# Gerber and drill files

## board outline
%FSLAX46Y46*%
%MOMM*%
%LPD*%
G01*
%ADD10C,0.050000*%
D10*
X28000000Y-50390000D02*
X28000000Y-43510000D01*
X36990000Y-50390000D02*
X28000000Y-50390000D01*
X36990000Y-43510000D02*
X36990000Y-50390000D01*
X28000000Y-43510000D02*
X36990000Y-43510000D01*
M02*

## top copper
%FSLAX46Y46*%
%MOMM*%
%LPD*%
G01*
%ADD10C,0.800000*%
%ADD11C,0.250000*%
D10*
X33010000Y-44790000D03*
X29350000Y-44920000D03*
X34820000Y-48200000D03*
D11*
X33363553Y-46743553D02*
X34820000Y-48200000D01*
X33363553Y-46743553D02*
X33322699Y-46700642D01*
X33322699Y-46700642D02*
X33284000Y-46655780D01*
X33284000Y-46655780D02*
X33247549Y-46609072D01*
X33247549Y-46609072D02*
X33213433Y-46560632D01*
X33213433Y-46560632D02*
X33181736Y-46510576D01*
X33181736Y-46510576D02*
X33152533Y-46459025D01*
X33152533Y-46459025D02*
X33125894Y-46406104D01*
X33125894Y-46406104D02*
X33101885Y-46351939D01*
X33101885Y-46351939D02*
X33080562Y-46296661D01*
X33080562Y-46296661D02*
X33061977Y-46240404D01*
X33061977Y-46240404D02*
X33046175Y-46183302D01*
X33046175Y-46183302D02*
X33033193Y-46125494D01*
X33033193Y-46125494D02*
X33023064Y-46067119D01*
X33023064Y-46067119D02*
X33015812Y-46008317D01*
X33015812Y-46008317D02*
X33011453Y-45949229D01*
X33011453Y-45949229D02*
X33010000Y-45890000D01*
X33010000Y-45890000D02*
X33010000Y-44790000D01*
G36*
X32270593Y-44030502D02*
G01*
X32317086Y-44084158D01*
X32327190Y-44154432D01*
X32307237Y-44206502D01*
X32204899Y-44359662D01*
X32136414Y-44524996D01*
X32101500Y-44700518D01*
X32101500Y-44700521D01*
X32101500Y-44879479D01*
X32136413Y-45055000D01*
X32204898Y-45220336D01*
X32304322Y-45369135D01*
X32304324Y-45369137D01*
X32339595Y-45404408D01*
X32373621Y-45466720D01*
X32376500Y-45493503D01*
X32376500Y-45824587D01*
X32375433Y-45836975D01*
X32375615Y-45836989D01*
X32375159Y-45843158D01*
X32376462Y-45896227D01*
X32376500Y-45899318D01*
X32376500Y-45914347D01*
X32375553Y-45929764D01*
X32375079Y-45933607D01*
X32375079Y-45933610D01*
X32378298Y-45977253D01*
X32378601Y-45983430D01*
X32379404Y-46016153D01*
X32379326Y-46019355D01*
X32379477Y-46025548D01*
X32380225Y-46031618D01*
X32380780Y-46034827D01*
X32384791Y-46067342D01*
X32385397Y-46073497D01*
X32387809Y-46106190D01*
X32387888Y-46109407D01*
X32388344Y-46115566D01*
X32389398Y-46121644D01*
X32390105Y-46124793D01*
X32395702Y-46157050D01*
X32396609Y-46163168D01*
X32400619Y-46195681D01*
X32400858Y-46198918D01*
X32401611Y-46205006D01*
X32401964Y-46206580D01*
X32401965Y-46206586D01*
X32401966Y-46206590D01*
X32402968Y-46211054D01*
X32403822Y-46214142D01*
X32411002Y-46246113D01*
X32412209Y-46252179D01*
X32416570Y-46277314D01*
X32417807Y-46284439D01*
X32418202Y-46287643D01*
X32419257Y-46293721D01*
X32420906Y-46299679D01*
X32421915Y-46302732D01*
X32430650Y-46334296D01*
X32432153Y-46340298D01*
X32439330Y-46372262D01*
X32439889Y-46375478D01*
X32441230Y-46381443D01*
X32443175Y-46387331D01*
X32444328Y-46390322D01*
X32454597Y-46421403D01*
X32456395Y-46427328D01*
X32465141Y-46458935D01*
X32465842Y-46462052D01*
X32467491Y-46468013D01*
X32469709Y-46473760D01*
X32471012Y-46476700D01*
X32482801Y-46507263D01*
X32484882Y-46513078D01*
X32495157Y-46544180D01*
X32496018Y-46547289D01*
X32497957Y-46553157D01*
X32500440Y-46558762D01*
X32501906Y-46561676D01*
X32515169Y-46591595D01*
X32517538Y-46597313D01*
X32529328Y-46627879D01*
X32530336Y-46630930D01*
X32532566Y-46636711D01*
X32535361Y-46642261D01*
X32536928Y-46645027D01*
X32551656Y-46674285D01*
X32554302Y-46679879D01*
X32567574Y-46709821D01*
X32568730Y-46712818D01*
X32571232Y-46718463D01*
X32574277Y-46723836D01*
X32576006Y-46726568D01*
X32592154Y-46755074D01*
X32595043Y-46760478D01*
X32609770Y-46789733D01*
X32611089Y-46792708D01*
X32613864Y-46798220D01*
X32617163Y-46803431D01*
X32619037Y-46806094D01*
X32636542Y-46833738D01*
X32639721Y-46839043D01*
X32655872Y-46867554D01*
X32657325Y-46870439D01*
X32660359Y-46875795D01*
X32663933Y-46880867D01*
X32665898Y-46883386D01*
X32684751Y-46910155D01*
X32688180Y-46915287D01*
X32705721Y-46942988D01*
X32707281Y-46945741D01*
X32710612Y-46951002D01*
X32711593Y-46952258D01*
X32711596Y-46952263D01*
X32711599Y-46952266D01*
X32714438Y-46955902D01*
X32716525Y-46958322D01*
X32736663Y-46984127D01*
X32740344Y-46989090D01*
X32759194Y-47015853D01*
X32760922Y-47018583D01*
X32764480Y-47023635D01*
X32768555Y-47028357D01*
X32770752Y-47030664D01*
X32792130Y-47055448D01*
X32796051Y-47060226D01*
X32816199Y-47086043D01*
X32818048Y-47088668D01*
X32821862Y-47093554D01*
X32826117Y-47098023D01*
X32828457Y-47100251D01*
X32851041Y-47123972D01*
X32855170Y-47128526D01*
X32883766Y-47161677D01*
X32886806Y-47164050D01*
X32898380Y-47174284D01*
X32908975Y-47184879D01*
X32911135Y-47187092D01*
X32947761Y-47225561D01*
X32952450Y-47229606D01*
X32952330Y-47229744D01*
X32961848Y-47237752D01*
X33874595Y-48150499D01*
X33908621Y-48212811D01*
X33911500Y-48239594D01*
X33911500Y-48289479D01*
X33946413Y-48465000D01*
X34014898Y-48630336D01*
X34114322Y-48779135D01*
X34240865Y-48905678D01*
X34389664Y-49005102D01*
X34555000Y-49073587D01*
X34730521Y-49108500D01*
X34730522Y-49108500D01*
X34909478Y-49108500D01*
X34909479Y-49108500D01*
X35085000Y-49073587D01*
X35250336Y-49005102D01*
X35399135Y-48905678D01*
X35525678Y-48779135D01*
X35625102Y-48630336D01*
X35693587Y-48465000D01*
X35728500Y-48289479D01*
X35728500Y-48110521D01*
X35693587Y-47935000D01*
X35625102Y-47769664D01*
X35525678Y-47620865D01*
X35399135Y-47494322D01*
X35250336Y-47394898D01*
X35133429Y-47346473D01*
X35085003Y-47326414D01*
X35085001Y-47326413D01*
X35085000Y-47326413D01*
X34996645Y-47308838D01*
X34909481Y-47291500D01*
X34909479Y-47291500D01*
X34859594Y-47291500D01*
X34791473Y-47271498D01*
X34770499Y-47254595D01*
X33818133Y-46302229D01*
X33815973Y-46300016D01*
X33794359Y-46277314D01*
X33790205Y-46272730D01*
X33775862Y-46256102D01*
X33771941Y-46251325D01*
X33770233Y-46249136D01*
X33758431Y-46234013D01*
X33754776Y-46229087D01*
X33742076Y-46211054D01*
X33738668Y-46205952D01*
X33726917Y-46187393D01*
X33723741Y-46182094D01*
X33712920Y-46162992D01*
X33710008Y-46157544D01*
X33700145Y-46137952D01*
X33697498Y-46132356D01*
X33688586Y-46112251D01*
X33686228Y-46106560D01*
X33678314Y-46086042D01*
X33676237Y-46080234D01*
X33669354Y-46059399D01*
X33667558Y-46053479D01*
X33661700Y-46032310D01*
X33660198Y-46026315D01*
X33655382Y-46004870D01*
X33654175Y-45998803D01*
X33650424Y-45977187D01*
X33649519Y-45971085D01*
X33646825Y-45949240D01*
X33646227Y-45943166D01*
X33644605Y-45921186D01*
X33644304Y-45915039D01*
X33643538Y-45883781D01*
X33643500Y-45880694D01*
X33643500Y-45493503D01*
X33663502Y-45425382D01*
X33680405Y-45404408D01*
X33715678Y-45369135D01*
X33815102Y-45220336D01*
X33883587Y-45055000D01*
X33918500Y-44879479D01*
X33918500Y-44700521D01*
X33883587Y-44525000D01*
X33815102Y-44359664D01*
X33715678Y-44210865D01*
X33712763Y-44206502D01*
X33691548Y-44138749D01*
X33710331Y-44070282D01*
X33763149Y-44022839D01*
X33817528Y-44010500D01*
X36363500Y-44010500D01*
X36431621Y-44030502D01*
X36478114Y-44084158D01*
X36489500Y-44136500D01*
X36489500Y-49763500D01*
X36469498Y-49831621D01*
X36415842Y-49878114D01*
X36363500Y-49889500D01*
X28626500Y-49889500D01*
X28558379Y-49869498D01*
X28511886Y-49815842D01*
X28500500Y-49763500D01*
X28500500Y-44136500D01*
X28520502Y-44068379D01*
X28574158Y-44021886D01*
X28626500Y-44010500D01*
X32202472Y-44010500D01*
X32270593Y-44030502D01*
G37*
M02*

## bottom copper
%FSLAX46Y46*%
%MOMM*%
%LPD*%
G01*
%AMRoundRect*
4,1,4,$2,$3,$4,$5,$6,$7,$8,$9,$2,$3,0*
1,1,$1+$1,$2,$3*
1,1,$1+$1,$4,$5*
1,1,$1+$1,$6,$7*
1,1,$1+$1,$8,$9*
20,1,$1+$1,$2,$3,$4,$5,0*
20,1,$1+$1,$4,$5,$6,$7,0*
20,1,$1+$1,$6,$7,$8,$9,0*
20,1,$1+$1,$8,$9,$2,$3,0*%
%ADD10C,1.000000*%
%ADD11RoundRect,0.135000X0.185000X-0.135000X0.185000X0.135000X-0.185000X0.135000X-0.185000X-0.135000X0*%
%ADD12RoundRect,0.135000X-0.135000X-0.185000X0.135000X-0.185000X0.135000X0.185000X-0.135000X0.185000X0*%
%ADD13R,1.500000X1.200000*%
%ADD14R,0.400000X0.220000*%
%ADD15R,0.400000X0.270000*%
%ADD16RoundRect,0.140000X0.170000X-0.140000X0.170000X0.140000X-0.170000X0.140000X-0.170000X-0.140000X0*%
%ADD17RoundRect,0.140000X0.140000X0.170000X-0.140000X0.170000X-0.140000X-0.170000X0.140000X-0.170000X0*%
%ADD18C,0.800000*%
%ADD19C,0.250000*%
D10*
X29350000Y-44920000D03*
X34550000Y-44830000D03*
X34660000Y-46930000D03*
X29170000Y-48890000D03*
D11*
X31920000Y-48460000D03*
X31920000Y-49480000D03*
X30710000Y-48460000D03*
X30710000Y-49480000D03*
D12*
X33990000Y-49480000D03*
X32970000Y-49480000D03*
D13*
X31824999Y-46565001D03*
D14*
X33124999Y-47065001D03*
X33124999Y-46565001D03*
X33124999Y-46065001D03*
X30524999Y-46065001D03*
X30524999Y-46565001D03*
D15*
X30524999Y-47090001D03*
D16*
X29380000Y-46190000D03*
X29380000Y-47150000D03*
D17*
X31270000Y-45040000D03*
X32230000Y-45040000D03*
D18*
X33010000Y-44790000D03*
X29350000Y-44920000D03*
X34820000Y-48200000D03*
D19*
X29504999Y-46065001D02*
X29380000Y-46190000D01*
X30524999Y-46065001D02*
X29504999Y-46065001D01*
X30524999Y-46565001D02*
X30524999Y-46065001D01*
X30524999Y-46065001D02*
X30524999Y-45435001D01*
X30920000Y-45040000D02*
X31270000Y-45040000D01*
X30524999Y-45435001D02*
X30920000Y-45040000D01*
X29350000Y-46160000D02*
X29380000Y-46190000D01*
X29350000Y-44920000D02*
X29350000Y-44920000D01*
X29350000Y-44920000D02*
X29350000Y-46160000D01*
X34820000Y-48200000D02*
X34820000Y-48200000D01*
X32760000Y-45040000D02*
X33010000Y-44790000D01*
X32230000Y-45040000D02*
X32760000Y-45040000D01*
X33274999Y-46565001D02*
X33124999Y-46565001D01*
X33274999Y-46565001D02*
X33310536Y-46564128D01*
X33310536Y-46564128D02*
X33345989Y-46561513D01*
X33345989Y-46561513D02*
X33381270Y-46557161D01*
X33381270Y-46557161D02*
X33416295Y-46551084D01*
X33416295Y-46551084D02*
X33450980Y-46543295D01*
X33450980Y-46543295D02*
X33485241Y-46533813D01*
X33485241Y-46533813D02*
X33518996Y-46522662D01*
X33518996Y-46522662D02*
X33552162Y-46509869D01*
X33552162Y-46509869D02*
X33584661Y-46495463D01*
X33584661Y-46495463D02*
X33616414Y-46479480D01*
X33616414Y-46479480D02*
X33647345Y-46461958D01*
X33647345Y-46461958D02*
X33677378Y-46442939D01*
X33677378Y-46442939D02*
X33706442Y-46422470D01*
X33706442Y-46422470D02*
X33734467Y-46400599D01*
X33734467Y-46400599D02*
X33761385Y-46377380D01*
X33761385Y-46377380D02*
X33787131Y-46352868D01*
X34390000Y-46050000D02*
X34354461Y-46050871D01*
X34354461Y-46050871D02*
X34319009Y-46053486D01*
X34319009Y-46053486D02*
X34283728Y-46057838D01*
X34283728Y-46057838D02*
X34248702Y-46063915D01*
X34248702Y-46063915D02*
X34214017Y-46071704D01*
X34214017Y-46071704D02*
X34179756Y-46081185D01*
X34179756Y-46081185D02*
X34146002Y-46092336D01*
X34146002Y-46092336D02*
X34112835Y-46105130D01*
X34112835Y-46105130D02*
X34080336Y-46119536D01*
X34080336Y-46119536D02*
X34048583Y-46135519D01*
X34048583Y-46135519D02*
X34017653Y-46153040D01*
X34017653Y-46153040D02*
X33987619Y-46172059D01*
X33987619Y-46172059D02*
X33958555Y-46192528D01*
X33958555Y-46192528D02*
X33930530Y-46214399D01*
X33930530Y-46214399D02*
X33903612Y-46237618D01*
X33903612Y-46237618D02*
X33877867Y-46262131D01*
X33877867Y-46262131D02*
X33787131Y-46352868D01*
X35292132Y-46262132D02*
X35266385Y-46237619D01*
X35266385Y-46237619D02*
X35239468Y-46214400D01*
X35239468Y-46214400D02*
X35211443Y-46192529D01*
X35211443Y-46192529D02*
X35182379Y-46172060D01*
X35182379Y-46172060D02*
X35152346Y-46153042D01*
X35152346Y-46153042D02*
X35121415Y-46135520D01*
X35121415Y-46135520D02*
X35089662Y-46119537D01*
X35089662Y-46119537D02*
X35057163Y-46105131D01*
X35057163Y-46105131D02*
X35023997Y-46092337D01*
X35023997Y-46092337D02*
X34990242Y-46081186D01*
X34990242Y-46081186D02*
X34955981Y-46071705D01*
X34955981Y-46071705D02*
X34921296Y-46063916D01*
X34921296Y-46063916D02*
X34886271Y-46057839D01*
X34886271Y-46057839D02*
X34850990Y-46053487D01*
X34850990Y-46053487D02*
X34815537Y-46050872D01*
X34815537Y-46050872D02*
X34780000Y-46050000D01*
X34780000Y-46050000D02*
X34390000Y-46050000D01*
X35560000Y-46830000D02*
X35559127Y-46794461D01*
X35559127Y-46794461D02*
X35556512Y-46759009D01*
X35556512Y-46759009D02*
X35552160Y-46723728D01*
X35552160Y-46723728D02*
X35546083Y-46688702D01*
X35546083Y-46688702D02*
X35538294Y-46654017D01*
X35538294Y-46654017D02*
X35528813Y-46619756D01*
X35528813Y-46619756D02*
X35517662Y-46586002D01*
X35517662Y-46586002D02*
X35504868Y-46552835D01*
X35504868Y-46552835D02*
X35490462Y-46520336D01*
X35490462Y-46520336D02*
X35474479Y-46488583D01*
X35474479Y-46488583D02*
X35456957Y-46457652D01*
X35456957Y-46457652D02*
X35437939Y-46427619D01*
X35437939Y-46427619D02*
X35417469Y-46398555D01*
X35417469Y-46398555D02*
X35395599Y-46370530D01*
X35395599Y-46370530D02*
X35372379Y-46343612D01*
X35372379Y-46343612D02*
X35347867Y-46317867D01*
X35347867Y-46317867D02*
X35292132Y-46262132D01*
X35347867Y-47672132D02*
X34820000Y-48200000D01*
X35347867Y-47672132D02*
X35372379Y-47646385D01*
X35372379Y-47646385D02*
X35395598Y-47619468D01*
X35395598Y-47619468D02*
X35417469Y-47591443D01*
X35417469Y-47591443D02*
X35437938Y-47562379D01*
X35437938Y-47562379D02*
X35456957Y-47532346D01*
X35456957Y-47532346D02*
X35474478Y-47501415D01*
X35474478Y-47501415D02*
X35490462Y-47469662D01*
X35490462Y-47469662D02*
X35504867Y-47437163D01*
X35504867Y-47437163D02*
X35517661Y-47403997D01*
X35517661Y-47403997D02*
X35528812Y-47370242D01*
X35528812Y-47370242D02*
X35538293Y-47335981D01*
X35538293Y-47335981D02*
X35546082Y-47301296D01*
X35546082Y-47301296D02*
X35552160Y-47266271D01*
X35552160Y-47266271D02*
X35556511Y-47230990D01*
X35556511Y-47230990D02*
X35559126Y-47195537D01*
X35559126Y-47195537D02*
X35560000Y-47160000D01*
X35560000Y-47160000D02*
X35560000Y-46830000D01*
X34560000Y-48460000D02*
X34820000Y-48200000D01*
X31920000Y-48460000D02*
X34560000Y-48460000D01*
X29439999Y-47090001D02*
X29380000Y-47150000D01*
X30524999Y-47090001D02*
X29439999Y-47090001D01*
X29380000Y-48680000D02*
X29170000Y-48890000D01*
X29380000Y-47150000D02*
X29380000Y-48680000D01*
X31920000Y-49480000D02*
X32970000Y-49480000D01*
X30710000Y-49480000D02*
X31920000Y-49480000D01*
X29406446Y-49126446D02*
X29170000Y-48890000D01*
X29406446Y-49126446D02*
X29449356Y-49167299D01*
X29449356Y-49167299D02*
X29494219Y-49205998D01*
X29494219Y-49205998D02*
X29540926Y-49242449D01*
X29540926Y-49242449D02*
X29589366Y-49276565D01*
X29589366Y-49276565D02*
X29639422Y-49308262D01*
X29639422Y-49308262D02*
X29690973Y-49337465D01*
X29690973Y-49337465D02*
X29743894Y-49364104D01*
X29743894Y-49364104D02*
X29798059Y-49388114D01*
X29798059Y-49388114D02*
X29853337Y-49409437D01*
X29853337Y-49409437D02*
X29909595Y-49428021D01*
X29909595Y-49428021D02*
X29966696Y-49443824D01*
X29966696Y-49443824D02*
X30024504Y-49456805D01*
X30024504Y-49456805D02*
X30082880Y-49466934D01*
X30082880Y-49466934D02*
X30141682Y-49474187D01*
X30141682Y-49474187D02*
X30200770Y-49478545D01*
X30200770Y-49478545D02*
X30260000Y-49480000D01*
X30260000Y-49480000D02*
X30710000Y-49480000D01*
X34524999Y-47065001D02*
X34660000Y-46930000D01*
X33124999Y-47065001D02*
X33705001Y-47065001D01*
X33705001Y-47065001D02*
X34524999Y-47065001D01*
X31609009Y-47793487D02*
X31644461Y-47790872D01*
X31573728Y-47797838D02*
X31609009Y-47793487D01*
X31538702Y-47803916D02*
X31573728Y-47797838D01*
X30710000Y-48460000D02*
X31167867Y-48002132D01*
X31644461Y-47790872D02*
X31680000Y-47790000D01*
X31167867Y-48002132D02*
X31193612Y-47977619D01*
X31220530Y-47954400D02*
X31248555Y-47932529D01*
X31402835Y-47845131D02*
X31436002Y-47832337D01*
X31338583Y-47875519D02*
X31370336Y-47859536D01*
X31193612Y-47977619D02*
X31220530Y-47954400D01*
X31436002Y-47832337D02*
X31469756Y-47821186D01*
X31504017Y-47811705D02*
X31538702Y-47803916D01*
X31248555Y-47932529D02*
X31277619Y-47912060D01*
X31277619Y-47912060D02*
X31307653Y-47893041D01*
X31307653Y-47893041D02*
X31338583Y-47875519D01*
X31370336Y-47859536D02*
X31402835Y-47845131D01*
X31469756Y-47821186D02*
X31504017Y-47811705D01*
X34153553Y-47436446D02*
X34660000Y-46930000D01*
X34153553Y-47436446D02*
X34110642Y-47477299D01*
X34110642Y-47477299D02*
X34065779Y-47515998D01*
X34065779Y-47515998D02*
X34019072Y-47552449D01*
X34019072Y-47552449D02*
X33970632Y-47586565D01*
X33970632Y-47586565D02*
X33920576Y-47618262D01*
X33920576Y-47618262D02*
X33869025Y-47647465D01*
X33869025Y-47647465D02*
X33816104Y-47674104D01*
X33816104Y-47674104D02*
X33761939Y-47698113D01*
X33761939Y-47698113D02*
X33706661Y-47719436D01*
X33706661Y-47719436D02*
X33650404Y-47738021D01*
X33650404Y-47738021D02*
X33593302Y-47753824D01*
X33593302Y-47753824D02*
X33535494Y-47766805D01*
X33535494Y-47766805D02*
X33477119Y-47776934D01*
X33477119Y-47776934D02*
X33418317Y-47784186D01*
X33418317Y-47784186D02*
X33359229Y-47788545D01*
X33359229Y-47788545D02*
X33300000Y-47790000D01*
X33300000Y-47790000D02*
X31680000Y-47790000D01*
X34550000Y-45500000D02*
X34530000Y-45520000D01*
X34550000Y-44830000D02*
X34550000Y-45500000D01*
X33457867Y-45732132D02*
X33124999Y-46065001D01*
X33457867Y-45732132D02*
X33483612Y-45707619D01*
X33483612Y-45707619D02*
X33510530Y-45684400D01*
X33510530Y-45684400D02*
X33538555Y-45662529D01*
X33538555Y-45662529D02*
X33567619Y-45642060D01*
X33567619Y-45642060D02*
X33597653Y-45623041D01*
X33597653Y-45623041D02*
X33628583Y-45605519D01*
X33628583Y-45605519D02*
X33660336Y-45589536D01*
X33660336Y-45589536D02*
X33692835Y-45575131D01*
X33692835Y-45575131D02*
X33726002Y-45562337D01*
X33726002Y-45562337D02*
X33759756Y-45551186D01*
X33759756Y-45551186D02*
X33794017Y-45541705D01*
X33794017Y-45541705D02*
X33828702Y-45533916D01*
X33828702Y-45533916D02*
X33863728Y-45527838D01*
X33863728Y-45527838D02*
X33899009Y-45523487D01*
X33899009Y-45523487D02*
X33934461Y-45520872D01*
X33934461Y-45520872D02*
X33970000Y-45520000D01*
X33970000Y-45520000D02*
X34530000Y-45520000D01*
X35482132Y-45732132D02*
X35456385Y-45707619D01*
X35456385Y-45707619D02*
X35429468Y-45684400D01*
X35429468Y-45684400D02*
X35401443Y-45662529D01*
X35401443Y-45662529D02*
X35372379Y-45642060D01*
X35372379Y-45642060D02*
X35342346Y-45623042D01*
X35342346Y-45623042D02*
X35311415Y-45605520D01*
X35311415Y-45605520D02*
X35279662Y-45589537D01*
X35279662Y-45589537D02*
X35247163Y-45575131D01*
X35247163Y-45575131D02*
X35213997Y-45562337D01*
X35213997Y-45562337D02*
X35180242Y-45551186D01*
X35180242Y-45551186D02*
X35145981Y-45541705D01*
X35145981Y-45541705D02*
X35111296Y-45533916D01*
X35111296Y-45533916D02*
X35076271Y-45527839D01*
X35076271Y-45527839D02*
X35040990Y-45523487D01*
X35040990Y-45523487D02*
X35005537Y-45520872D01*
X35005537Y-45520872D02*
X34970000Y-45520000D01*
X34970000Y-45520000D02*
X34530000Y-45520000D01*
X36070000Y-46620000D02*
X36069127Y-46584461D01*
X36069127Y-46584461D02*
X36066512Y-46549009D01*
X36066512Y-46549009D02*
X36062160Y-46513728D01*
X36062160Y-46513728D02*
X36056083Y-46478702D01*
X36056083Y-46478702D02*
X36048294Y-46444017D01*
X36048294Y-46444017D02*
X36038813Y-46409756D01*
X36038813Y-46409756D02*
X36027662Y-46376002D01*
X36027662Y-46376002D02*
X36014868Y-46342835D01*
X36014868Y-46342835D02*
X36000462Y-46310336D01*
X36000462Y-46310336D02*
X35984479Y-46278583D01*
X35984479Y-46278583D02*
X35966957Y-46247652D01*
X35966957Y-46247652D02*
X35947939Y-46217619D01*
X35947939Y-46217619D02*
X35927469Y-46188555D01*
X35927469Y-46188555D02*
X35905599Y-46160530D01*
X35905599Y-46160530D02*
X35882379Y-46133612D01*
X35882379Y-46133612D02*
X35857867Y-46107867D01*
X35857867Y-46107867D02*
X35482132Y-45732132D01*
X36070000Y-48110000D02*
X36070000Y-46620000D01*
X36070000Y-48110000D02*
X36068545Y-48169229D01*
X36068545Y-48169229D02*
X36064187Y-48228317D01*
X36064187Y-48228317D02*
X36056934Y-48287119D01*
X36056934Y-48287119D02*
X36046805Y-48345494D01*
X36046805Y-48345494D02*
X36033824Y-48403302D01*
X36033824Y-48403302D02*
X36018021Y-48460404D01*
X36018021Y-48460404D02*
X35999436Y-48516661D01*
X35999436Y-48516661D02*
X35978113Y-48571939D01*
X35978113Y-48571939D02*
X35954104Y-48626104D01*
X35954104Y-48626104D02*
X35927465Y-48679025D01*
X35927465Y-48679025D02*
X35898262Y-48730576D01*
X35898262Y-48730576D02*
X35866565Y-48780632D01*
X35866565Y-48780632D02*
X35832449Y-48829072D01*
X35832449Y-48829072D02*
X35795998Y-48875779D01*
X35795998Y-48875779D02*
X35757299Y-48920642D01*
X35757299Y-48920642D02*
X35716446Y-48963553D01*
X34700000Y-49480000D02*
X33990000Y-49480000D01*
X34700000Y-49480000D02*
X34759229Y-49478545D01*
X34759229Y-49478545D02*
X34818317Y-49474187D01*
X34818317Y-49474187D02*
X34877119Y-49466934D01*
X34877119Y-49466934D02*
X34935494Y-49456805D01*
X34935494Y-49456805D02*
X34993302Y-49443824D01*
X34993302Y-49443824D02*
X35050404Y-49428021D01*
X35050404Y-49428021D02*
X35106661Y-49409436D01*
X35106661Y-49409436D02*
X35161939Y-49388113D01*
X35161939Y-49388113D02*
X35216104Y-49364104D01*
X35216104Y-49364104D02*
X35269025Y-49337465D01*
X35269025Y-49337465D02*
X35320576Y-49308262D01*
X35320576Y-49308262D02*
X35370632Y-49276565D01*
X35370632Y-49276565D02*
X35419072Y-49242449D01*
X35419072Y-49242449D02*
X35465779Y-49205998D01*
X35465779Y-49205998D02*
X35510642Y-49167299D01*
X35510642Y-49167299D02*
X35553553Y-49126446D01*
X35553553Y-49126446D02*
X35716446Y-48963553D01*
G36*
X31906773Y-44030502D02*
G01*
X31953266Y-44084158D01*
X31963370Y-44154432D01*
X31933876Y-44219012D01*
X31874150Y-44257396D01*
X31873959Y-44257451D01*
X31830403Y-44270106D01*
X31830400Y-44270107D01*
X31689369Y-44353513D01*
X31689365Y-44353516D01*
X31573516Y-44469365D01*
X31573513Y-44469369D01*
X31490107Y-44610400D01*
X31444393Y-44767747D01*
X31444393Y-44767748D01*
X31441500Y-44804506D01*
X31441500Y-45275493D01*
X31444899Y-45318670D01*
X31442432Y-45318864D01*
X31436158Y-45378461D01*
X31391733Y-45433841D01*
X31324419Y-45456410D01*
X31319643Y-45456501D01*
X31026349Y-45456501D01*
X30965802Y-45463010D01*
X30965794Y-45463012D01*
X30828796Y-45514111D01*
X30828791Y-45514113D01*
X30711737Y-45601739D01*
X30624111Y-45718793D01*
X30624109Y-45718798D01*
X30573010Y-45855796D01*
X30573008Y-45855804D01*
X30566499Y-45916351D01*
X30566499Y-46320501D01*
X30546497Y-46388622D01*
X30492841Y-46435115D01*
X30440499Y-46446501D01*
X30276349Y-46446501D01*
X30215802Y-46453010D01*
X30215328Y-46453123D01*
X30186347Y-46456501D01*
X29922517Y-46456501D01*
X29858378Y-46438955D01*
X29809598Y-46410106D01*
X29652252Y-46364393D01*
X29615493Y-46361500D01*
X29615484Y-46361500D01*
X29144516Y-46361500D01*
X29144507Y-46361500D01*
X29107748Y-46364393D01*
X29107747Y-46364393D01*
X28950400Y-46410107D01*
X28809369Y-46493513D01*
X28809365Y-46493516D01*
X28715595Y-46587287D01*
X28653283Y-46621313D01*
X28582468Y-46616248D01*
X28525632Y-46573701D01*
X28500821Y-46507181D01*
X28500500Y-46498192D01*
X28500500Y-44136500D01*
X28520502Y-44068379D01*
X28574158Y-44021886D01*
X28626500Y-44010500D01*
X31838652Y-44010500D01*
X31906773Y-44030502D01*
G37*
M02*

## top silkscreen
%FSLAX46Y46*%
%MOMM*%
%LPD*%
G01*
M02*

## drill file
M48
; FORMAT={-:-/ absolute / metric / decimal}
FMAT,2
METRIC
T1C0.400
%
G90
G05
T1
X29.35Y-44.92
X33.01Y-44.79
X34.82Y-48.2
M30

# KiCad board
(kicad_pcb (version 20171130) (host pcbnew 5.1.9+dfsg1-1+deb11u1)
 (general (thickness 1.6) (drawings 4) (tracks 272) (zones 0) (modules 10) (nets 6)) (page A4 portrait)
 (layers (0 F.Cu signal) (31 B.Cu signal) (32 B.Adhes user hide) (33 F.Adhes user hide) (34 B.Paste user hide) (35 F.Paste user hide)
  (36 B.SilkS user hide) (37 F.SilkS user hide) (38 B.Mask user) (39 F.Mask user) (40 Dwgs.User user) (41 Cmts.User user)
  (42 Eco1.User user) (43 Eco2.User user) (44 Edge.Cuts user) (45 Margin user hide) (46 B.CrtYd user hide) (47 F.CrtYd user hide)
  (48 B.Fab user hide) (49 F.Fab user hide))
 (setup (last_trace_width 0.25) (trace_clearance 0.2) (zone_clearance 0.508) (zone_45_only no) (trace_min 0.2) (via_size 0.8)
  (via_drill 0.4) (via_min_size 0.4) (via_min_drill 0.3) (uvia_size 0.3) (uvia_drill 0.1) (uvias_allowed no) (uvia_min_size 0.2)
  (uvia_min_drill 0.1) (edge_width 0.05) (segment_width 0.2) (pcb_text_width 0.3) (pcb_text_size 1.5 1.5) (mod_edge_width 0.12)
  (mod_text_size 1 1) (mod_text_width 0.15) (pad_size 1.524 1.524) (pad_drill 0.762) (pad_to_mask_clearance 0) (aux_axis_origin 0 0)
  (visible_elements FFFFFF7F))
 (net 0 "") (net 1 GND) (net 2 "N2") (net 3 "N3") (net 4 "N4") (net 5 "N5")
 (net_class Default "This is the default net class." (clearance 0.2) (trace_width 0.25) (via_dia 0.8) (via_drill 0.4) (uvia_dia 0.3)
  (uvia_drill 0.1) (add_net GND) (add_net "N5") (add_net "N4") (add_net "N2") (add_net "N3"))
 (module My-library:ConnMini (layer B.Cu) (at 29.35 44.92)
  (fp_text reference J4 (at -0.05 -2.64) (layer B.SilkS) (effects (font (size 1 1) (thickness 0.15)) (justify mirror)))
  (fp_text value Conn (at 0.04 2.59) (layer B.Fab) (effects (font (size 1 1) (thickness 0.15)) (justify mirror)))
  (pad 1 smd circle (at 0 0) (size 1 1) (layers B.Cu B.Paste B.Mask) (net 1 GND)))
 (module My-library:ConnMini (layer B.Cu) (at 34.55 44.83)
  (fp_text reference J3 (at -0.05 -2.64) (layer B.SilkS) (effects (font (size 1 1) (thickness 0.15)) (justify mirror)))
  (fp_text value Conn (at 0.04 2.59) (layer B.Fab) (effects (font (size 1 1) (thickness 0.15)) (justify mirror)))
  (pad 1 smd circle (at 0 0) (size 1 1) (layers B.Cu B.Paste B.Mask) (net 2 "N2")))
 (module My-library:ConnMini (layer B.Cu) (at 34.66 46.93)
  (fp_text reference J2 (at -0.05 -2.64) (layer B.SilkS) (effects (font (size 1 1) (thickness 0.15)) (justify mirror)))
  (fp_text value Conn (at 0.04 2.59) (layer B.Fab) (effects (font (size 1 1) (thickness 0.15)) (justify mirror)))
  (pad 1 smd circle (at 0 0) (size 1 1) (layers B.Cu B.Paste B.Mask) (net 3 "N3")))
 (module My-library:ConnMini (layer B.Cu) (at 29.17 48.89)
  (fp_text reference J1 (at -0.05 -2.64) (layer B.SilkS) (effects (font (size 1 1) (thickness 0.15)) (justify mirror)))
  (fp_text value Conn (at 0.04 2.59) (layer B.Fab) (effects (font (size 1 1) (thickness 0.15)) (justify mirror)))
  (pad 1 smd circle (at 0 0) (size 1 1) (layers B.Cu B.Paste B.Mask) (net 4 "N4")))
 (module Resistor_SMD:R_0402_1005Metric (layer B.Cu) (at 31.92 48.97 90)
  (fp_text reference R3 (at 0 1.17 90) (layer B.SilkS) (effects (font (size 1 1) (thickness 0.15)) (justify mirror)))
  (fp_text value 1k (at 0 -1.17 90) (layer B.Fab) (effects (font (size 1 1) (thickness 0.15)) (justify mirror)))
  (pad 2 smd roundrect (at 0.51 0 90) (size 0.54 0.64) (layers B.Cu B.Paste B.Mask) (roundrect_rratio 0.25) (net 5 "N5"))
  (pad 1 smd roundrect (at -0.51 0 90) (size 0.54 0.64) (layers B.Cu B.Paste B.Mask) (roundrect_rratio 0.25) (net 4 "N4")))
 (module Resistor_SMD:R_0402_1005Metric (layer B.Cu) (at 30.71 48.97 90)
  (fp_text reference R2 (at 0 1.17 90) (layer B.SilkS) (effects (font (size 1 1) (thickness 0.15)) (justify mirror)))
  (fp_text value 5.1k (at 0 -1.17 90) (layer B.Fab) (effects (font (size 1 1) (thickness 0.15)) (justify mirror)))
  (pad 2 smd roundrect (at 0.51 0 90) (size 0.54 0.64) (layers B.Cu B.Paste B.Mask) (roundrect_rratio 0.25) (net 3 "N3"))
  (pad 1 smd roundrect (at -0.51 0 90) (size 0.54 0.64) (layers B.Cu B.Paste B.Mask) (roundrect_rratio 0.25) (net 4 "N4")))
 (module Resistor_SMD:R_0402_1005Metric (layer B.Cu) (at 33.48 49.48)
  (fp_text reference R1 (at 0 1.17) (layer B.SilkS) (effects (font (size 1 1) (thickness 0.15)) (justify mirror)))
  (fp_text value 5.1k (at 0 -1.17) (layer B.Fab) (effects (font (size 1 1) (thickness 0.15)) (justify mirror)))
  (pad 2 smd roundrect (at 0.51 0) (size 0.54 0.64) (layers B.Cu B.Paste B.Mask) (roundrect_rratio 0.25) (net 2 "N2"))
  (pad 1 smd roundrect (at -0.51 0) (size 0.54 0.64) (layers B.Cu B.Paste B.Mask) (roundrect_rratio 0.25) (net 4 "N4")))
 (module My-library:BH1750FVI (layer B.Cu) (at 31.824999 46.565001)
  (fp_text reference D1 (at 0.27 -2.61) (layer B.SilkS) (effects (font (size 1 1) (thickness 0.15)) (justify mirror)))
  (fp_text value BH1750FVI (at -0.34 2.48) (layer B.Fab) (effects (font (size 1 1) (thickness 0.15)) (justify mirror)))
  (pad 7 smd rect (at 0 0) (size 1.5 1.2) (layers B.Cu B.Paste B.Mask))
  (pad 6 smd rect (at 1.3 0.5) (size 0.4 0.22) (layers B.Cu B.Paste B.Mask) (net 3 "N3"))
  (pad 5 smd rect (at 1.3 0) (size 0.4 0.22) (layers B.Cu B.Paste B.Mask) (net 5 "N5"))
  (pad 4 smd rect (at 1.3 -0.5) (size 0.4 0.22) (layers B.Cu B.Paste B.Mask) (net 2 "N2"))
  (pad 3 smd rect (at -1.3 -0.5) (size 0.4 0.22) (layers B.Cu B.Paste B.Mask) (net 1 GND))
  (pad 2 smd rect (at -1.3 0) (size 0.4 0.22) (layers B.Cu B.Paste B.Mask) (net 1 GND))
  (pad 1 smd rect (at -1.3 0.525) (size 0.4 0.27) (layers B.Cu B.Paste B.Mask) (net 4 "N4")))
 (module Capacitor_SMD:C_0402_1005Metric (layer B.Cu) (at 29.38 46.67 90)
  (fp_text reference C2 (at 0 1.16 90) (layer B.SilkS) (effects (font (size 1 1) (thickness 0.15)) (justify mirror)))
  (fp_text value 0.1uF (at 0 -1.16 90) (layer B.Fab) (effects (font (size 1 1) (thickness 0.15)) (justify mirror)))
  (pad 2 smd roundrect (at 0.48 0 90) (size 0.56 0.62) (layers B.Cu B.Paste B.Mask) (roundrect_rratio 0.25) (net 1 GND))
  (pad 1 smd roundrect (at -0.48 0 90) (size 0.56 0.62) (layers B.Cu B.Paste B.Mask) (roundrect_rratio 0.25) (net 4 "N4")))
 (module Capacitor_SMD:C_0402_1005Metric (layer B.Cu) (at 31.75 45.04 180)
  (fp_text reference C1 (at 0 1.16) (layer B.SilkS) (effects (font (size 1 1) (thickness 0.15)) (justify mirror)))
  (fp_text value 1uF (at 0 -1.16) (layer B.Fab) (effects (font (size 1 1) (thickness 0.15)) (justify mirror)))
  (pad 2 smd roundrect (at 0.48 0 180) (size 0.56 0.62) (layers B.Cu B.Paste B.Mask) (roundrect_rratio 0.25) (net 1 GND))
  (pad 1 smd roundrect (at -0.48 0 180) (size 0.56 0.62) (layers B.Cu B.Paste B.Mask) (roundrect_rratio 0.25) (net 5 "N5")))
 (gr_line (start 28 50.39) (end 28 43.51) (layer Edge.Cuts) (width 0.05))
 (gr_line (start 36.99 50.39) (end 28 50.39) (layer Edge.Cuts) (width 0.05))
 (gr_line (start 36.99 43.51) (end 36.99 50.39) (layer Edge.Cuts) (width 0.05))
 (gr_line (start 28 43.51) (end 36.99 43.51) (layer Edge.Cuts) (width 0.05))
 (via (at 33.01 44.79) (size 0.8) (drill 0.4) (layers F.Cu B.Cu) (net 5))
 (segment (start 29.504999 46.065001) (end 29.38 46.19) (width 0.25) (layer B.Cu) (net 1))
 (segment (start 30.524999 46.065001) (end 29.504999 46.065001) (width 0.25) (layer B.Cu) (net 1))
 (segment (start 30.524999 46.565001) (end 30.524999 46.065001) (width 0.25) (layer B.Cu) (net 1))
 (segment (start 30.524999 46.065001) (end 30.524999 45.435001) (width 0.25) (layer B.Cu) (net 1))
 (segment (start 30.92 45.04) (end 31.27 45.04) (width 0.25) (layer B.Cu) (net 1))
 (segment (start 30.524999 45.435001) (end 30.92 45.04) (width 0.25) (layer B.Cu) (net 1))
 (segment (start 29.35 46.16) (end 29.38 46.19) (width 0.25) (layer B.Cu) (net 1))
 (segment (start 29.35 44.92) (end 29.35 44.92) (width 0.25) (layer B.Cu) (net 1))
 (segment (start 29.35 44.92) (end 29.35 46.16) (width 0.25) (layer B.Cu) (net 1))
 (via (at 29.35 44.92) (size 0.8) (drill 0.4) (layers F.Cu B.Cu) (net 1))
 (segment (start 34.82 48.2) (end 34.82 48.2) (width 0.25) (layer B.Cu) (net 5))
 (via (at 34.82 48.2) (size 0.8) (drill 0.4) (layers F.Cu B.Cu) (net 5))
 (segment (start 32.76 45.04) (end 33.01 44.79) (width 0.25) (layer B.Cu) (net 5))
 (segment (start 32.23 45.04) (end 32.76 45.04) (width 0.25) (layer B.Cu) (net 5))
 (segment (start 33.363553 46.743553) (end 34.82 48.2) (width 0.25) (layer F.Cu) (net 5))
 (segment (start 33.363553 46.743553) (end 33.322699 46.700642) (width 0.25) (layer F.Cu) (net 5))
 (segment (start 33.322699 46.700642) (end 33.284 46.65578) (width 0.25) (layer F.Cu) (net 5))
 (segment (start 33.284 46.65578) (end 33.247549 46.609072) (width 0.25) (layer F.Cu) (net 5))
 (segment (start 33.247549 46.609072) (end 33.213433 46.560632) (width 0.25) (layer F.Cu) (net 5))
 (segment (start 33.213433 46.560632) (end 33.181736 46.510576) (width 0.25) (layer F.Cu) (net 5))
 (segment (start 33.181736 46.510576) (end 33.152533 46.459025) (width 0.25) (layer F.Cu) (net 5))
 (segment (start 33.152533 46.459025) (end 33.125894 46.406104) (width 0.25) (layer F.Cu) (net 5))
 (segment (start 33.125894 46.406104) (end 33.101885 46.351939) (width 0.25) (layer F.Cu) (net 5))
 (segment (start 33.101885 46.351939) (end 33.080562 46.296661) (width 0.25) (layer F.Cu) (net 5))
 (segment (start 33.080562 46.296661) (end 33.061977 46.240404) (width 0.25) (layer F.Cu) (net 5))
 (segment (start 33.061977 46.240404) (end 33.046175 46.183302) (width 0.25) (layer F.Cu) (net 5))
 (segment (start 33.046175 46.183302) (end 33.033193 46.125494) (width 0.25) (layer F.Cu) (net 5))
 (segment (start 33.033193 46.125494) (end 33.023064 46.067119) (width 0.25) (layer F.Cu) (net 5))
 (segment (start 33.023064 46.067119) (end 33.015812 46.008317) (width 0.25) (layer F.Cu) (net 5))
 (segment (start 33.015812 46.008317) (end 33.011453 45.949229) (width 0.25) (layer F.Cu) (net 5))
 (segment (start 33.011453 45.949229) (end 33.01 45.89) (width 0.25) (layer F.Cu) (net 5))
 (segment (start 33.01 45.89) (end 33.01 44.79) (width 0.25) (layer F.Cu) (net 5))
 (segment (start 33.274999 46.565001) (end 33.124999 46.565001) (width 0.25) (layer B.Cu) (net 5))
 (segment (start 33.274999 46.565001) (end 33.310536 46.564128) (width 0.25) (layer B.Cu) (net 5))
 (segment (start 33.310536 46.564128) (end 33.345989 46.561513) (width 0.25) (layer B.Cu) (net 5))
 (segment (start 33.345989 46.561513) (end 33.38127 46.557161) (width 0.25) (layer B.Cu) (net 5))
 (segment (start 33.38127 46.557161) (end 33.416295 46.551084) (width 0.25) (layer B.Cu) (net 5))
 (segment (start 33.416295 46.551084) (end 33.45098 46.543295) (width 0.25) (layer B.Cu) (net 5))
 (segment (start 33.45098 46.543295) (end 33.485241 46.533813) (width 0.25) (layer B.Cu) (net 5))
 (segment (start 33.485241 46.533813) (end 33.518996 46.522662) (width 0.25) (layer B.Cu) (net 5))
 (segment (start 33.518996 46.522662) (end 33.552162 46.509869) (width 0.25) (layer B.Cu) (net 5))
 (segment (start 33.552162 46.509869) (end 33.584661 46.495463) (width 0.25) (layer B.Cu) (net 5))
 (segment (start 33.584661 46.495463) (end 33.616414 46.47948) (width 0.25) (layer B.Cu) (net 5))
 (segment (start 33.616414 46.47948) (end 33.647345 46.461958) (width 0.25) (layer B.Cu) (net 5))
 (segment (start 33.647345 46.461958) (end 33.677378 46.442939) (width 0.25) (layer B.Cu) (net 5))
 (segment (start 33.677378 46.442939) (end 33.706442 46.42247) (width 0.25) (layer B.Cu) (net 5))
 (segment (start 33.706442 46.42247) (end 33.734467 46.400599) (width 0.25) (layer B.Cu) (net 5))
 (segment (start 33.734467 46.400599) (end 33.761385 46.37738) (width 0.25) (layer B.Cu) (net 5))
 (segment (start 33.761385 46.37738) (end 33.787131 46.352868) (width 0.25) (layer B.Cu) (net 5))
 (segment (start 34.39 46.05) (end 34.354461 46.050871) (width 0.25) (layer B.Cu) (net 5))
 (segment (start 34.354461 46.050871) (end 34.319009 46.053486) (width 0.25) (layer B.Cu) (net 5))
 (segment (start 34.319009 46.053486) (end 34.283728 46.057838) (width 0.25) (layer B.Cu) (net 5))
 (segment (start 34.283728 46.057838) (end 34.248702 46.063915) (width 0.25) (layer B.Cu) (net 5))
 (segment (start 34.248702 46.063915) (end 34.214017 46.071704) (width 0.25) (layer B.Cu) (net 5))
 (segment (start 34.214017 46.071704) (end 34.179756 46.081185) (width 0.25) (layer B.Cu) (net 5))
 (segment (start 34.179756 46.081185) (end 34.146002 46.092336) (width 0.25) (layer B.Cu) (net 5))
 (segment (start 34.146002 46.092336) (end 34.112835 46.10513) (width 0.25) (layer B.Cu) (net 5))
 (segment (start 34.112835 46.10513) (end 34.080336 46.119536) (width 0.25) (layer B.Cu) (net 5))
 (segment (start 34.080336 46.119536) (end 34.048583 46.135519) (width 0.25) (layer B.Cu) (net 5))
 (segment (start 34.048583 46.135519) (end 34.017653 46.15304) (width 0.25) (layer B.Cu) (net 5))
 (segment (start 34.017653 46.15304) (end 33.987619 46.172059) (width 0.25) (layer B.Cu) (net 5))
 (segment (start 33.987619 46.172059) (end 33.958555 46.192528) (width 0.25) (layer B.Cu) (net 5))
 (segment (start 33.958555 46.192528) (end 33.93053 46.214399) (width 0.25) (layer B.Cu) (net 5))
 (segment (start 33.93053 46.214399) (end 33.903612 46.237618) (width 0.25) (layer B.Cu) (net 5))
 (segment (start 33.903612 46.237618) (end 33.877867 46.262131) (width 0.25) (layer B.Cu) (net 5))
 (segment (start 33.877867 46.262131) (end 33.787131 46.352868) (width 0.25) (layer B.Cu) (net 5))
 (segment (start 35.292132 46.262132) (end 35.266385 46.237619) (width 0.25) (layer B.Cu) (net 5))
 (segment (start 35.266385 46.237619) (end 35.239468 46.2144) (width 0.25) (layer B.Cu) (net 5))
 (segment (start 35.239468 46.2144) (end 35.211443 46.192529) (width 0.25) (layer B.Cu) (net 5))
 (segment (start 35.211443 46.192529) (end 35.182379 46.17206) (width 0.25) (layer B.Cu) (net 5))
 (segment (start 35.182379 46.17206) (end 35.152346 46.153042) (width 0.25) (layer B.Cu) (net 5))
 (segment (start 35.152346 46.153042) (end 35.121415 46.13552) (width 0.25) (layer B.Cu) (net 5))
 (segment (start 35.121415 46.13552) (end 35.089662 46.119537) (width 0.25) (layer B.Cu) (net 5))
 (segment (start 35.089662 46.119537) (end 35.057163 46.105131) (width 0.25) (layer B.Cu) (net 5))
 (segment (start 35.057163 46.105131) (end 35.023997 46.092337) (width 0.25) (layer B.Cu) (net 5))
 (segment (start 35.023997 46.092337) (end 34.990242 46.081186) (width 0.25) (layer B.Cu) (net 5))
 (segment (start 34.990242 46.081186) (end 34.955981 46.071705) (width 0.25) (layer B.Cu) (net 5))
 (segment (start 34.955981 46.071705) (end 34.921296 46.063916) (width 0.25) (layer B.Cu) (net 5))
 (segment (start 34.921296 46.063916) (end 34.886271 46.057839) (width 0.25) (layer B.Cu) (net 5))
 (segment (start 34.886271 46.057839) (end 34.85099 46.053487) (width 0.25) (layer B.Cu) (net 5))
 (segment (start 34.85099 46.053487) (end 34.815537 46.050872) (width 0.25) (layer B.Cu) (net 5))
 (segment (start 34.815537 46.050872) (end 34.78 46.05) (width 0.25) (layer B.Cu) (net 5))
 (segment (start 34.78 46.05) (end 34.39 46.05) (width 0.25) (layer B.Cu) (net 5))
 (segment (start 35.56 46.83) (end 35.559127 46.794461) (width 0.25) (layer B.Cu) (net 5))
 (segment (start 35.559127 46.794461) (end 35.556512 46.759009) (width 0.25) (layer B.Cu) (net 5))
 (segment (start 35.556512 46.759009) (end 35.55216 46.723728) (width 0.25) (layer B.Cu) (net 5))
 (segment (start 35.55216 46.723728) (end 35.546083 46.688702) (width 0.25) (layer B.Cu) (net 5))
 (segment (start 35.546083 46.688702) (end 35.538294 46.654017) (width 0.25) (layer B.Cu) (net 5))
 (segment (start 35.538294 46.654017) (end 35.528813 46.619756) (width 0.25) (layer B.Cu) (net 5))
 (segment (start 35.528813 46.619756) (end 35.517662 46.586002) (width 0.25) (layer B.Cu) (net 5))
 (segment (start 35.517662 46.586002) (end 35.504868 46.552835) (width 0.25) (layer B.Cu) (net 5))
 (segment (start 35.504868 46.552835) (end 35.490462 46.520336) (width 0.25) (layer B.Cu) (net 5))
 (segment (start 35.490462 46.520336) (end 35.474479 46.488583) (width 0.25) (layer B.Cu) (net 5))
 (segment (start 35.474479 46.488583) (end 35.456957 46.457652) (width 0.25) (layer B.Cu) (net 5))
 (segment (start 35.456957 46.457652) (end 35.437939 46.427619) (width 0.25) (layer B.Cu) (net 5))
 (segment (start 35.437939 46.427619) (end 35.417469 46.398555) (width 0.25) (layer B.Cu) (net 5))
 (segment (start 35.417469 46.398555) (end 35.395599 46.37053) (width 0.25) (layer B.Cu) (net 5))
 (segment (start 35.395599 46.37053) (end 35.372379 46.343612) (width 0.25) (layer B.Cu) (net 5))
 (segment (start 35.372379 46.343612) (end 35.347867 46.317867) (width 0.25) (layer B.Cu) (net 5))
 (segment (start 35.347867 46.317867) (end 35.292132 46.262132) (width 0.25) (layer B.Cu) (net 5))
 (segment (start 35.347867 47.672132) (end 34.82 48.2) (width 0.25) (layer B.Cu) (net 5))
 (segment (start 35.347867 47.672132) (end 35.372379 47.646385) (width 0.25) (layer B.Cu) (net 5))
 (segment (start 35.372379 47.646385) (end 35.395598 47.619468) (width 0.25) (layer B.Cu) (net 5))
 (segment (start 35.395598 47.619468) (end 35.417469 47.591443) (width 0.25) (layer B.Cu) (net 5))
 (segment (start 35.417469 47.591443) (end 35.437938 47.562379) (width 0.25) (layer B.Cu) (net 5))
 (segment (start 35.437938 47.562379) (end 35.456957 47.532346) (width 0.25) (layer B.Cu) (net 5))
 (segment (start 35.456957 47.532346) (end 35.474478 47.501415) (width 0.25) (layer B.Cu) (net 5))
 (segment (start 35.474478 47.501415) (end 35.490462 47.469662) (width 0.25) (layer B.Cu) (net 5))
 (segment (start 35.490462 47.469662) (end 35.504867 47.437163) (width 0.25) (layer B.Cu) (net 5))
 (segment (start 35.504867 47.437163) (end 35.517661 47.403997) (width 0.25) (layer B.Cu) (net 5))
 (segment (start 35.517661 47.403997) (end 35.528812 47.370242) (width 0.25) (layer B.Cu) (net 5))
 (segment (start 35.528812 47.370242) (end 35.538293 47.335981) (width 0.25) (layer B.Cu) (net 5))
 (segment (start 35.538293 47.335981) (end 35.546082 47.301296) (width 0.25) (layer B.Cu) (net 5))
 (segment (start 35.546082 47.301296) (end 35.55216 47.266271) (width 0.25) (layer B.Cu) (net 5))
 (segment (start 35.55216 47.266271) (end 35.556511 47.23099) (width 0.25) (layer B.Cu) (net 5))
 (segment (start 35.556511 47.23099) (end 35.559126 47.195537) (width 0.25) (layer B.Cu) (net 5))
 (segment (start 35.559126 47.195537) (end 35.56 47.16) (width 0.25) (layer B.Cu) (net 5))
 (segment (start 35.56 47.16) (end 35.56 46.83) (width 0.25) (layer B.Cu) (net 5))
 (segment (start 34.56 48.46) (end 34.82 48.2) (width 0.25) (layer B.Cu) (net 5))
 (segment (start 31.92 48.46) (end 34.56 48.46) (width 0.25) (layer B.Cu) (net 5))
 (segment (start 29.439999 47.090001) (end 29.38 47.15) (width 0.25) (layer B.Cu) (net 4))
 (segment (start 30.524999 47.090001) (end 29.439999 47.090001) (width 0.25) (layer B.Cu) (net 4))
 (segment (start 29.38 48.68) (end 29.17 48.89) (width 0.25) (layer B.Cu) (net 4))
 (segment (start 29.38 47.15) (end 29.38 48.68) (width 0.25) (layer B.Cu) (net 4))
 (segment (start 31.92 49.48) (end 32.97 49.48) (width 0.25) (layer B.Cu) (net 4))
 (segment (start 30.71 49.48) (end 31.92 49.48) (width 0.25) (layer B.Cu) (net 4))
 (segment (start 29.406446 49.126446) (end 29.17 48.89) (width 0.25) (layer B.Cu) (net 4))
 (segment (start 29.406446 49.126446) (end 29.449356 49.167299) (width 0.25) (layer B.Cu) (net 4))
 (segment (start 29.449356 49.167299) (end 29.494219 49.205998) (width 0.25) (layer B.Cu) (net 4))
 (segment (start 29.494219 49.205998) (end 29.540926 49.242449) (width 0.25) (layer B.Cu) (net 4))
 (segment (start 29.540926 49.242449) (end 29.589366 49.276565) (width 0.25) (layer B.Cu) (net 4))
 (segment (start 29.589366 49.276565) (end 29.639422 49.308262) (width 0.25) (layer B.Cu) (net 4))
 (segment (start 29.639422 49.308262) (end 29.690973 49.337465) (width 0.25) (layer B.Cu) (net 4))
 (segment (start 29.690973 49.337465) (end 29.743894 49.364104) (width 0.25) (layer B.Cu) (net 4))
 (segment (start 29.743894 49.364104) (end 29.798059 49.388114) (width 0.25) (layer B.Cu) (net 4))
 (segment (start 29.798059 49.388114) (end 29.853337 49.409437) (width 0.25) (layer B.Cu) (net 4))
 (segment (start 29.853337 49.409437) (end 29.909595 49.428021) (width 0.25) (layer B.Cu) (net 4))
 (segment (start 29.909595 49.428021) (end 29.966696 49.443824) (width 0.25) (layer B.Cu) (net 4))
 (segment (start 29.966696 49.443824) (end 30.024504 49.456805) (width 0.25) (layer B.Cu) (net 4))
 (segment (start 30.024504 49.456805) (end 30.08288 49.466934) (width 0.25) (layer B.Cu) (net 4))
 (segment (start 30.08288 49.466934) (end 30.141682 49.474187) (width 0.25) (layer B.Cu) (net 4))
 (segment (start 30.141682 49.474187) (end 30.20077 49.478545) (width 0.25) (layer B.Cu) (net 4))
 (segment (start 30.20077 49.478545) (end 30.26 49.48) (width 0.25) (layer B.Cu) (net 4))
 (segment (start 30.26 49.48) (end 30.71 49.48) (width 0.25) (layer B.Cu) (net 4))
 (segment (start 34.524999 47.065001) (end 34.66 46.93) (width 0.25) (layer B.Cu) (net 3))
 (segment (start 33.124999 47.065001) (end 33.705001 47.065001) (width 0.25) (layer B.Cu) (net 3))
 (segment (start 33.705001 47.065001) (end 34.524999 47.065001) (width 0.25) (layer B.Cu) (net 3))
 (segment (start 31.609009 47.793487) (end 31.644461 47.790872) (width 0.25) (layer B.Cu) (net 3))
 (segment (start 31.573728 47.797838) (end 31.609009 47.793487) (width 0.25) (layer B.Cu) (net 3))
 (segment (start 31.538702 47.803916) (end 31.573728 47.797838) (width 0.25) (layer B.Cu) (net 3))
 (segment (start 30.71 48.46) (end 31.167867 48.002132) (width 0.25) (layer B.Cu) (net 3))
 (segment (start 31.644461 47.790872) (end 31.68 47.79) (width 0.25) (layer B.Cu) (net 3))
 (segment (start 31.167867 48.002132) (end 31.193612 47.977619) (width 0.25) (layer B.Cu) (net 3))
 (segment (start 31.22053 47.9544) (end 31.248555 47.932529) (width 0.25) (layer B.Cu) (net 3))
 (segment (start 31.402835 47.845131) (end 31.436002 47.832337) (width 0.25) (layer B.Cu) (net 3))
 (segment (start 31.338583 47.875519) (end 31.370336 47.859536) (width 0.25) (layer B.Cu) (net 3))
 (segment (start 31.193612 47.977619) (end 31.22053 47.9544) (width 0.25) (layer B.Cu) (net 3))
 (segment (start 31.436002 47.832337) (end 31.469756 47.821186) (width 0.25) (layer B.Cu) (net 3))
 (segment (start 31.504017 47.811705) (end 31.538702 47.803916) (width 0.25) (layer B.Cu) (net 3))
 (segment (start 31.248555 47.932529) (end 31.277619 47.91206) (width 0.25) (layer B.Cu) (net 3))
 (segment (start 31.277619 47.91206) (end 31.307653 47.893041) (width 0.25) (layer B.Cu) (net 3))
 (segment (start 31.307653 47.893041) (end 31.338583 47.875519) (width 0.25) (layer B.Cu) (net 3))
 (segment (start 31.370336 47.859536) (end 31.402835 47.845131) (width 0.25) (layer B.Cu) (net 3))
 (segment (start 31.469756 47.821186) (end 31.504017 47.811705) (width 0.25) (layer B.Cu) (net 3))
 (segment (start 34.153553 47.436446) (end 34.66 46.93) (width 0.25) (layer B.Cu) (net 3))
 (segment (start 34.153553 47.436446) (end 34.110642 47.477299) (width 0.25) (layer B.Cu) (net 3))
 (segment (start 34.110642 47.477299) (end 34.065779 47.515998) (width 0.25) (layer B.Cu) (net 3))
 (segment (start 34.065779 47.515998) (end 34.019072 47.552449) (width 0.25) (layer B.Cu) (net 3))
 (segment (start 34.019072 47.552449) (end 33.970632 47.586565) (width 0.25) (layer B.Cu) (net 3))
 (segment (start 33.970632 47.586565) (end 33.920576 47.618262) (width 0.25) (layer B.Cu) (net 3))
 (segment (start 33.920576 47.618262) (end 33.869025 47.647465) (width 0.25) (layer B.Cu) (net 3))
 (segment (start 33.869025 47.647465) (end 33.816104 47.674104) (width 0.25) (layer B.Cu) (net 3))
 (segment (start 33.816104 47.674104) (end 33.761939 47.698113) (width 0.25) (layer B.Cu) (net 3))
 (segment (start 33.761939 47.698113) (end 33.706661 47.719436) (width 0.25) (layer B.Cu) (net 3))
 (segment (start 33.706661 47.719436) (end 33.650404 47.738021) (width 0.25) (layer B.Cu) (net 3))
 (segment (start 33.650404 47.738021) (end 33.593302 47.753824) (width 0.25) (layer B.Cu) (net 3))
 (segment (start 33.593302 47.753824) (end 33.535494 47.766805) (width 0.25) (layer B.Cu) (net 3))
 (segment (start 33.535494 47.766805) (end 33.477119 47.776934) (width 0.25) (layer B.Cu) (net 3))
 (segment (start 33.477119 47.776934) (end 33.418317 47.784186) (width 0.25) (layer B.Cu) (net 3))
 (segment (start 33.418317 47.784186) (end 33.359229 47.788545) (width 0.25) (layer B.Cu) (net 3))
 (segment (start 33.359229 47.788545) (end 33.3 47.79) (width 0.25) (layer B.Cu) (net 3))
 (segment (start 33.3 47.79) (end 31.68 47.79) (width 0.25) (layer B.Cu) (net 3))
 (segment (start 34.55 45.5) (end 34.53 45.52) (width 0.25) (layer B.Cu) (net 2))
 (segment (start 34.55 44.83) (end 34.55 45.5) (width 0.25) (layer B.Cu) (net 2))
 (segment (start 33.457867 45.732132) (end 33.124999 46.065001) (width 0.25) (layer B.Cu) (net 2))
 (segment (start 33.457867 45.732132) (end 33.483612 45.707619) (width 0.25) (layer B.Cu) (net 2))
 (segment (start 33.483612 45.707619) (end 33.51053 45.6844) (width 0.25) (layer B.Cu) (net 2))
 (segment (start 33.51053 45.6844) (end 33.538555 45.662529) (width 0.25) (layer B.Cu) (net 2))
 (segment (start 33.538555 45.662529) (end 33.567619 45.64206) (width 0.25) (layer B.Cu) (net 2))
 (segment (start 33.567619 45.64206) (end 33.597653 45.623041) (width 0.25) (layer B.Cu) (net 2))
 (segment (start 33.597653 45.623041) (end 33.628583 45.605519) (width 0.25) (layer B.Cu) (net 2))
 (segment (start 33.628583 45.605519) (end 33.660336 45.589536) (width 0.25) (layer B.Cu) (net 2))
 (segment (start 33.660336 45.589536) (end 33.692835 45.575131) (width 0.25) (layer B.Cu) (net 2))
 (segment (start 33.692835 45.575131) (end 33.726002 45.562337) (width 0.25) (layer B.Cu) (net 2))
 (segment (start 33.726002 45.562337) (end 33.759756 45.551186) (width 0.25) (layer B.Cu) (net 2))
 (segment (start 33.759756 45.551186) (end 33.794017 45.541705) (width 0.25) (layer B.Cu) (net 2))
 (segment (start 33.794017 45.541705) (end 33.828702 45.533916) (width 0.25) (layer B.Cu) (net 2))
 (segment (start 33.828702 45.533916) (end 33.863728 45.527838) (width 0.25) (layer B.Cu) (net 2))
 (segment (start 33.863728 45.527838) (end 33.899009 45.523487) (width 0.25) (layer B.Cu) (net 2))
 (segment (start 33.899009 45.523487) (end 33.934461 45.520872) (width 0.25) (layer B.Cu) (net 2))
 (segment (start 33.934461 45.520872) (end 33.97 45.52) (width 0.25) (layer B.Cu) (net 2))
 (segment (start 33.97 45.52) (end 34.53 45.52) (width 0.25) (layer B.Cu) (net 2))
 (segment (start 35.482132 45.732132) (end 35.456385 45.707619) (width 0.25) (layer B.Cu) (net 2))
 (segment (start 35.456385 45.707619) (end 35.429468 45.6844) (width 0.25) (layer B.Cu) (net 2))
 (segment (start 35.429468 45.6844) (end 35.401443 45.662529) (width 0.25) (layer B.Cu) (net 2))
 (segment (start 35.401443 45.662529) (end 35.372379 45.64206) (width 0.25) (layer B.Cu) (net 2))
 (segment (start 35.372379 45.64206) (end 35.342346 45.623042) (width 0.25) (layer B.Cu) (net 2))
 (segment (start 35.342346 45.623042) (end 35.311415 45.60552) (width 0.25) (layer B.Cu) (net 2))
 (segment (start 35.311415 45.60552) (end 35.279662 45.589537) (width 0.25) (layer B.Cu) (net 2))
 (segment (start 35.279662 45.589537) (end 35.247163 45.575131) (width 0.25) (layer B.Cu) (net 2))
 (segment (start 35.247163 45.575131) (end 35.213997 45.562337) (width 0.25) (layer B.Cu) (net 2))
 (segment (start 35.213997 45.562337) (end 35.180242 45.551186) (width 0.25) (layer B.Cu) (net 2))
 (segment (start 35.180242 45.551186) (end 35.145981 45.541705) (width 0.25) (layer B.Cu) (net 2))
 (segment (start 35.145981 45.541705) (end 35.111296 45.533916) (width 0.25) (layer B.Cu) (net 2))
 (segment (start 35.111296 45.533916) (end 35.076271 45.527839) (width 0.25) (layer B.Cu) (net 2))
 (segment (start 35.076271 45.527839) (end 35.04099 45.523487) (width 0.25) (layer B.Cu) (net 2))
 (segment (start 35.04099 45.523487) (end 35.005537 45.520872) (width 0.25) (layer B.Cu) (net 2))
 (segment (start 35.005537 45.520872) (end 34.97 45.52) (width 0.25) (layer B.Cu) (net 2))
 (segment (start 34.97 45.52) (end 34.53 45.52) (width 0.25) (layer B.Cu) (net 2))
 (segment (start 36.07 46.62) (end 36.069127 46.584461) (width 0.25) (layer B.Cu) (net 2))
 (segment (start 36.069127 46.584461) (end 36.066512 46.549009) (width 0.25) (layer B.Cu) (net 2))
 (segment (start 36.066512 46.549009) (end 36.06216 46.513728) (width 0.25) (layer B.Cu) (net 2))
 (segment (start 36.06216 46.513728) (end 36.056083 46.478702) (width 0.25) (layer B.Cu) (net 2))
 (segment (start 36.056083 46.478702) (end 36.048294 46.444017) (width 0.25) (layer B.Cu) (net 2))
 (segment (start 36.048294 46.444017) (end 36.038813 46.409756) (width 0.25) (layer B.Cu) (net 2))
 (segment (start 36.038813 46.409756) (end 36.027662 46.376002) (width 0.25) (layer B.Cu) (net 2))
 (segment (start 36.027662 46.376002) (end 36.014868 46.342835) (width 0.25) (layer B.Cu) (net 2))
 (segment (start 36.014868 46.342835) (end 36.000462 46.310336) (width 0.25) (layer B.Cu) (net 2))
 (segment (start 36.000462 46.310336) (end 35.984479 46.278583) (width 0.25) (layer B.Cu) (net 2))
 (segment (start 35.984479 46.278583) (end 35.966957 46.247652) (width 0.25) (layer B.Cu) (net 2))
 (segment (start 35.966957 46.247652) (end 35.947939 46.217619) (width 0.25) (layer B.Cu) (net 2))
 (segment (start 35.947939 46.217619) (end 35.927469 46.188555) (width 0.25) (layer B.Cu) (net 2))
 (segment (start 35.927469 46.188555) (end 35.905599 46.16053) (width 0.25) (layer B.Cu) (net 2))
 (segment (start 35.905599 46.16053) (end 35.882379 46.133612) (width 0.25) (layer B.Cu) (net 2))
 (segment (start 35.882379 46.133612) (end 35.857867 46.107867) (width 0.25) (layer B.Cu) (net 2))
 (segment (start 35.857867 46.107867) (end 35.482132 45.732132) (width 0.25) (layer B.Cu) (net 2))
 (segment (start 36.07 48.11) (end 36.07 46.62) (width 0.25) (layer B.Cu) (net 2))
 (segment (start 36.07 48.11) (end 36.068545 48.169229) (width 0.25) (layer B.Cu) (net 2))
 (segment (start 36.068545 48.169229) (end 36.064187 48.228317) (width 0.25) (layer B.Cu) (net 2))
 (segment (start 36.064187 48.228317) (end 36.056934 48.287119) (width 0.25) (layer B.Cu) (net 2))
 (segment (start 36.056934 48.287119) (end 36.046805 48.345494) (width 0.25) (layer B.Cu) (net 2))
 (segment (start 36.046805 48.345494) (end 36.033824 48.403302) (width 0.25) (layer B.Cu) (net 2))
 (segment (start 36.033824 48.403302) (end 36.018021 48.460404) (width 0.25) (layer B.Cu) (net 2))
 (segment (start 36.018021 48.460404) (end 35.999436 48.516661) (width 0.25) (layer B.Cu) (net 2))
 (segment (start 35.999436 48.516661) (end 35.978113 48.571939) (width 0.25) (layer B.Cu) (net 2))
 (segment (start 35.978113 48.571939) (end 35.954104 48.626104) (width 0.25) (layer B.Cu) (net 2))
 (segment (start 35.954104 48.626104) (end 35.927465 48.679025) (width 0.25) (layer B.Cu) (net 2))
 (segment (start 35.927465 48.679025) (end 35.898262 48.730576) (width 0.25) (layer B.Cu) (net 2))
 (segment (start 35.898262 48.730576) (end 35.866565 48.780632) (width 0.25) (layer B.Cu) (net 2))
 (segment (start 35.866565 48.780632) (end 35.832449 48.829072) (width 0.25) (layer B.Cu) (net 2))
 (segment (start 35.832449 48.829072) (end 35.795998 48.875779) (width 0.25) (layer B.Cu) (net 2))
 (segment (start 35.795998 48.875779) (end 35.757299 48.920642) (width 0.25) (layer B.Cu) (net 2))
 (segment (start 35.757299 48.920642) (end 35.716446 48.963553) (width 0.25) (layer B.Cu) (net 2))
 (segment (start 34.7 49.48) (end 33.99 49.48) (width 0.25) (layer B.Cu) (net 2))
 (segment (start 34.7 49.48) (end 34.759229 49.478545) (width 0.25) (layer B.Cu) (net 2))
 (segment (start 34.759229 49.478545) (end 34.818317 49.474187) (width 0.25) (layer B.Cu) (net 2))
 (segment (start 34.818317 49.474187) (end 34.877119 49.466934) (width 0.25) (layer B.Cu) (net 2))
 (segment (start 34.877119 49.466934) (end 34.935494 49.456805) (width 0.25) (layer B.Cu) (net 2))
 (segment (start 34.935494 49.456805) (end 34.993302 49.443824) (width 0.25) (layer B.Cu) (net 2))
 (segment (start 34.993302 49.443824) (end 35.050404 49.428021) (width 0.25) (layer B.Cu) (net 2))
 (segment (start 35.050404 49.428021) (end 35.106661 49.409436) (width 0.25) (layer B.Cu) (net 2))
 (segment (start 35.106661 49.409436) (end 35.161939 49.388113) (width 0.25) (layer B.Cu) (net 2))
 (segment (start 35.161939 49.388113) (end 35.216104 49.364104) (width 0.25) (layer B.Cu) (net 2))
 (segment (start 35.216104 49.364104) (end 35.269025 49.337465) (width 0.25) (layer B.Cu) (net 2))
 (segment (start 35.269025 49.337465) (end 35.320576 49.308262) (width 0.25) (layer B.Cu) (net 2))
 (segment (start 35.320576 49.308262) (end 35.370632 49.276565) (width 0.25) (layer B.Cu) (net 2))
 (segment (start 35.370632 49.276565) (end 35.419072 49.242449) (width 0.25) (layer B.Cu) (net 2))
 (segment (start 35.419072 49.242449) (end 35.465779 49.205998) (width 0.25) (layer B.Cu) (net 2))
 (segment (start 35.465779 49.205998) (end 35.510642 49.167299) (width 0.25) (layer B.Cu) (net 2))
 (segment (start 35.510642 49.167299) (end 35.553553 49.126446) (width 0.25) (layer B.Cu) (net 2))
 (segment (start 35.553553 49.126446) (end 35.716446 48.963553) (width 0.25) (layer B.Cu) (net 2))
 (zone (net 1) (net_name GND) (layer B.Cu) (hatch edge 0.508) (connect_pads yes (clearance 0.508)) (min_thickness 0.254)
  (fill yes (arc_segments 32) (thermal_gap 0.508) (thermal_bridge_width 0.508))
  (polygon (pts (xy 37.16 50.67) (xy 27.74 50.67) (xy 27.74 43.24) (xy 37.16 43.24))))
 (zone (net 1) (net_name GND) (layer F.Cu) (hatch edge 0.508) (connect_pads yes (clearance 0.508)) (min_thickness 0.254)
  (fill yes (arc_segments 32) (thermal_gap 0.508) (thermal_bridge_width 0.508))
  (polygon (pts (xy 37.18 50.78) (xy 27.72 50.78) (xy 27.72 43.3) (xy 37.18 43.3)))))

